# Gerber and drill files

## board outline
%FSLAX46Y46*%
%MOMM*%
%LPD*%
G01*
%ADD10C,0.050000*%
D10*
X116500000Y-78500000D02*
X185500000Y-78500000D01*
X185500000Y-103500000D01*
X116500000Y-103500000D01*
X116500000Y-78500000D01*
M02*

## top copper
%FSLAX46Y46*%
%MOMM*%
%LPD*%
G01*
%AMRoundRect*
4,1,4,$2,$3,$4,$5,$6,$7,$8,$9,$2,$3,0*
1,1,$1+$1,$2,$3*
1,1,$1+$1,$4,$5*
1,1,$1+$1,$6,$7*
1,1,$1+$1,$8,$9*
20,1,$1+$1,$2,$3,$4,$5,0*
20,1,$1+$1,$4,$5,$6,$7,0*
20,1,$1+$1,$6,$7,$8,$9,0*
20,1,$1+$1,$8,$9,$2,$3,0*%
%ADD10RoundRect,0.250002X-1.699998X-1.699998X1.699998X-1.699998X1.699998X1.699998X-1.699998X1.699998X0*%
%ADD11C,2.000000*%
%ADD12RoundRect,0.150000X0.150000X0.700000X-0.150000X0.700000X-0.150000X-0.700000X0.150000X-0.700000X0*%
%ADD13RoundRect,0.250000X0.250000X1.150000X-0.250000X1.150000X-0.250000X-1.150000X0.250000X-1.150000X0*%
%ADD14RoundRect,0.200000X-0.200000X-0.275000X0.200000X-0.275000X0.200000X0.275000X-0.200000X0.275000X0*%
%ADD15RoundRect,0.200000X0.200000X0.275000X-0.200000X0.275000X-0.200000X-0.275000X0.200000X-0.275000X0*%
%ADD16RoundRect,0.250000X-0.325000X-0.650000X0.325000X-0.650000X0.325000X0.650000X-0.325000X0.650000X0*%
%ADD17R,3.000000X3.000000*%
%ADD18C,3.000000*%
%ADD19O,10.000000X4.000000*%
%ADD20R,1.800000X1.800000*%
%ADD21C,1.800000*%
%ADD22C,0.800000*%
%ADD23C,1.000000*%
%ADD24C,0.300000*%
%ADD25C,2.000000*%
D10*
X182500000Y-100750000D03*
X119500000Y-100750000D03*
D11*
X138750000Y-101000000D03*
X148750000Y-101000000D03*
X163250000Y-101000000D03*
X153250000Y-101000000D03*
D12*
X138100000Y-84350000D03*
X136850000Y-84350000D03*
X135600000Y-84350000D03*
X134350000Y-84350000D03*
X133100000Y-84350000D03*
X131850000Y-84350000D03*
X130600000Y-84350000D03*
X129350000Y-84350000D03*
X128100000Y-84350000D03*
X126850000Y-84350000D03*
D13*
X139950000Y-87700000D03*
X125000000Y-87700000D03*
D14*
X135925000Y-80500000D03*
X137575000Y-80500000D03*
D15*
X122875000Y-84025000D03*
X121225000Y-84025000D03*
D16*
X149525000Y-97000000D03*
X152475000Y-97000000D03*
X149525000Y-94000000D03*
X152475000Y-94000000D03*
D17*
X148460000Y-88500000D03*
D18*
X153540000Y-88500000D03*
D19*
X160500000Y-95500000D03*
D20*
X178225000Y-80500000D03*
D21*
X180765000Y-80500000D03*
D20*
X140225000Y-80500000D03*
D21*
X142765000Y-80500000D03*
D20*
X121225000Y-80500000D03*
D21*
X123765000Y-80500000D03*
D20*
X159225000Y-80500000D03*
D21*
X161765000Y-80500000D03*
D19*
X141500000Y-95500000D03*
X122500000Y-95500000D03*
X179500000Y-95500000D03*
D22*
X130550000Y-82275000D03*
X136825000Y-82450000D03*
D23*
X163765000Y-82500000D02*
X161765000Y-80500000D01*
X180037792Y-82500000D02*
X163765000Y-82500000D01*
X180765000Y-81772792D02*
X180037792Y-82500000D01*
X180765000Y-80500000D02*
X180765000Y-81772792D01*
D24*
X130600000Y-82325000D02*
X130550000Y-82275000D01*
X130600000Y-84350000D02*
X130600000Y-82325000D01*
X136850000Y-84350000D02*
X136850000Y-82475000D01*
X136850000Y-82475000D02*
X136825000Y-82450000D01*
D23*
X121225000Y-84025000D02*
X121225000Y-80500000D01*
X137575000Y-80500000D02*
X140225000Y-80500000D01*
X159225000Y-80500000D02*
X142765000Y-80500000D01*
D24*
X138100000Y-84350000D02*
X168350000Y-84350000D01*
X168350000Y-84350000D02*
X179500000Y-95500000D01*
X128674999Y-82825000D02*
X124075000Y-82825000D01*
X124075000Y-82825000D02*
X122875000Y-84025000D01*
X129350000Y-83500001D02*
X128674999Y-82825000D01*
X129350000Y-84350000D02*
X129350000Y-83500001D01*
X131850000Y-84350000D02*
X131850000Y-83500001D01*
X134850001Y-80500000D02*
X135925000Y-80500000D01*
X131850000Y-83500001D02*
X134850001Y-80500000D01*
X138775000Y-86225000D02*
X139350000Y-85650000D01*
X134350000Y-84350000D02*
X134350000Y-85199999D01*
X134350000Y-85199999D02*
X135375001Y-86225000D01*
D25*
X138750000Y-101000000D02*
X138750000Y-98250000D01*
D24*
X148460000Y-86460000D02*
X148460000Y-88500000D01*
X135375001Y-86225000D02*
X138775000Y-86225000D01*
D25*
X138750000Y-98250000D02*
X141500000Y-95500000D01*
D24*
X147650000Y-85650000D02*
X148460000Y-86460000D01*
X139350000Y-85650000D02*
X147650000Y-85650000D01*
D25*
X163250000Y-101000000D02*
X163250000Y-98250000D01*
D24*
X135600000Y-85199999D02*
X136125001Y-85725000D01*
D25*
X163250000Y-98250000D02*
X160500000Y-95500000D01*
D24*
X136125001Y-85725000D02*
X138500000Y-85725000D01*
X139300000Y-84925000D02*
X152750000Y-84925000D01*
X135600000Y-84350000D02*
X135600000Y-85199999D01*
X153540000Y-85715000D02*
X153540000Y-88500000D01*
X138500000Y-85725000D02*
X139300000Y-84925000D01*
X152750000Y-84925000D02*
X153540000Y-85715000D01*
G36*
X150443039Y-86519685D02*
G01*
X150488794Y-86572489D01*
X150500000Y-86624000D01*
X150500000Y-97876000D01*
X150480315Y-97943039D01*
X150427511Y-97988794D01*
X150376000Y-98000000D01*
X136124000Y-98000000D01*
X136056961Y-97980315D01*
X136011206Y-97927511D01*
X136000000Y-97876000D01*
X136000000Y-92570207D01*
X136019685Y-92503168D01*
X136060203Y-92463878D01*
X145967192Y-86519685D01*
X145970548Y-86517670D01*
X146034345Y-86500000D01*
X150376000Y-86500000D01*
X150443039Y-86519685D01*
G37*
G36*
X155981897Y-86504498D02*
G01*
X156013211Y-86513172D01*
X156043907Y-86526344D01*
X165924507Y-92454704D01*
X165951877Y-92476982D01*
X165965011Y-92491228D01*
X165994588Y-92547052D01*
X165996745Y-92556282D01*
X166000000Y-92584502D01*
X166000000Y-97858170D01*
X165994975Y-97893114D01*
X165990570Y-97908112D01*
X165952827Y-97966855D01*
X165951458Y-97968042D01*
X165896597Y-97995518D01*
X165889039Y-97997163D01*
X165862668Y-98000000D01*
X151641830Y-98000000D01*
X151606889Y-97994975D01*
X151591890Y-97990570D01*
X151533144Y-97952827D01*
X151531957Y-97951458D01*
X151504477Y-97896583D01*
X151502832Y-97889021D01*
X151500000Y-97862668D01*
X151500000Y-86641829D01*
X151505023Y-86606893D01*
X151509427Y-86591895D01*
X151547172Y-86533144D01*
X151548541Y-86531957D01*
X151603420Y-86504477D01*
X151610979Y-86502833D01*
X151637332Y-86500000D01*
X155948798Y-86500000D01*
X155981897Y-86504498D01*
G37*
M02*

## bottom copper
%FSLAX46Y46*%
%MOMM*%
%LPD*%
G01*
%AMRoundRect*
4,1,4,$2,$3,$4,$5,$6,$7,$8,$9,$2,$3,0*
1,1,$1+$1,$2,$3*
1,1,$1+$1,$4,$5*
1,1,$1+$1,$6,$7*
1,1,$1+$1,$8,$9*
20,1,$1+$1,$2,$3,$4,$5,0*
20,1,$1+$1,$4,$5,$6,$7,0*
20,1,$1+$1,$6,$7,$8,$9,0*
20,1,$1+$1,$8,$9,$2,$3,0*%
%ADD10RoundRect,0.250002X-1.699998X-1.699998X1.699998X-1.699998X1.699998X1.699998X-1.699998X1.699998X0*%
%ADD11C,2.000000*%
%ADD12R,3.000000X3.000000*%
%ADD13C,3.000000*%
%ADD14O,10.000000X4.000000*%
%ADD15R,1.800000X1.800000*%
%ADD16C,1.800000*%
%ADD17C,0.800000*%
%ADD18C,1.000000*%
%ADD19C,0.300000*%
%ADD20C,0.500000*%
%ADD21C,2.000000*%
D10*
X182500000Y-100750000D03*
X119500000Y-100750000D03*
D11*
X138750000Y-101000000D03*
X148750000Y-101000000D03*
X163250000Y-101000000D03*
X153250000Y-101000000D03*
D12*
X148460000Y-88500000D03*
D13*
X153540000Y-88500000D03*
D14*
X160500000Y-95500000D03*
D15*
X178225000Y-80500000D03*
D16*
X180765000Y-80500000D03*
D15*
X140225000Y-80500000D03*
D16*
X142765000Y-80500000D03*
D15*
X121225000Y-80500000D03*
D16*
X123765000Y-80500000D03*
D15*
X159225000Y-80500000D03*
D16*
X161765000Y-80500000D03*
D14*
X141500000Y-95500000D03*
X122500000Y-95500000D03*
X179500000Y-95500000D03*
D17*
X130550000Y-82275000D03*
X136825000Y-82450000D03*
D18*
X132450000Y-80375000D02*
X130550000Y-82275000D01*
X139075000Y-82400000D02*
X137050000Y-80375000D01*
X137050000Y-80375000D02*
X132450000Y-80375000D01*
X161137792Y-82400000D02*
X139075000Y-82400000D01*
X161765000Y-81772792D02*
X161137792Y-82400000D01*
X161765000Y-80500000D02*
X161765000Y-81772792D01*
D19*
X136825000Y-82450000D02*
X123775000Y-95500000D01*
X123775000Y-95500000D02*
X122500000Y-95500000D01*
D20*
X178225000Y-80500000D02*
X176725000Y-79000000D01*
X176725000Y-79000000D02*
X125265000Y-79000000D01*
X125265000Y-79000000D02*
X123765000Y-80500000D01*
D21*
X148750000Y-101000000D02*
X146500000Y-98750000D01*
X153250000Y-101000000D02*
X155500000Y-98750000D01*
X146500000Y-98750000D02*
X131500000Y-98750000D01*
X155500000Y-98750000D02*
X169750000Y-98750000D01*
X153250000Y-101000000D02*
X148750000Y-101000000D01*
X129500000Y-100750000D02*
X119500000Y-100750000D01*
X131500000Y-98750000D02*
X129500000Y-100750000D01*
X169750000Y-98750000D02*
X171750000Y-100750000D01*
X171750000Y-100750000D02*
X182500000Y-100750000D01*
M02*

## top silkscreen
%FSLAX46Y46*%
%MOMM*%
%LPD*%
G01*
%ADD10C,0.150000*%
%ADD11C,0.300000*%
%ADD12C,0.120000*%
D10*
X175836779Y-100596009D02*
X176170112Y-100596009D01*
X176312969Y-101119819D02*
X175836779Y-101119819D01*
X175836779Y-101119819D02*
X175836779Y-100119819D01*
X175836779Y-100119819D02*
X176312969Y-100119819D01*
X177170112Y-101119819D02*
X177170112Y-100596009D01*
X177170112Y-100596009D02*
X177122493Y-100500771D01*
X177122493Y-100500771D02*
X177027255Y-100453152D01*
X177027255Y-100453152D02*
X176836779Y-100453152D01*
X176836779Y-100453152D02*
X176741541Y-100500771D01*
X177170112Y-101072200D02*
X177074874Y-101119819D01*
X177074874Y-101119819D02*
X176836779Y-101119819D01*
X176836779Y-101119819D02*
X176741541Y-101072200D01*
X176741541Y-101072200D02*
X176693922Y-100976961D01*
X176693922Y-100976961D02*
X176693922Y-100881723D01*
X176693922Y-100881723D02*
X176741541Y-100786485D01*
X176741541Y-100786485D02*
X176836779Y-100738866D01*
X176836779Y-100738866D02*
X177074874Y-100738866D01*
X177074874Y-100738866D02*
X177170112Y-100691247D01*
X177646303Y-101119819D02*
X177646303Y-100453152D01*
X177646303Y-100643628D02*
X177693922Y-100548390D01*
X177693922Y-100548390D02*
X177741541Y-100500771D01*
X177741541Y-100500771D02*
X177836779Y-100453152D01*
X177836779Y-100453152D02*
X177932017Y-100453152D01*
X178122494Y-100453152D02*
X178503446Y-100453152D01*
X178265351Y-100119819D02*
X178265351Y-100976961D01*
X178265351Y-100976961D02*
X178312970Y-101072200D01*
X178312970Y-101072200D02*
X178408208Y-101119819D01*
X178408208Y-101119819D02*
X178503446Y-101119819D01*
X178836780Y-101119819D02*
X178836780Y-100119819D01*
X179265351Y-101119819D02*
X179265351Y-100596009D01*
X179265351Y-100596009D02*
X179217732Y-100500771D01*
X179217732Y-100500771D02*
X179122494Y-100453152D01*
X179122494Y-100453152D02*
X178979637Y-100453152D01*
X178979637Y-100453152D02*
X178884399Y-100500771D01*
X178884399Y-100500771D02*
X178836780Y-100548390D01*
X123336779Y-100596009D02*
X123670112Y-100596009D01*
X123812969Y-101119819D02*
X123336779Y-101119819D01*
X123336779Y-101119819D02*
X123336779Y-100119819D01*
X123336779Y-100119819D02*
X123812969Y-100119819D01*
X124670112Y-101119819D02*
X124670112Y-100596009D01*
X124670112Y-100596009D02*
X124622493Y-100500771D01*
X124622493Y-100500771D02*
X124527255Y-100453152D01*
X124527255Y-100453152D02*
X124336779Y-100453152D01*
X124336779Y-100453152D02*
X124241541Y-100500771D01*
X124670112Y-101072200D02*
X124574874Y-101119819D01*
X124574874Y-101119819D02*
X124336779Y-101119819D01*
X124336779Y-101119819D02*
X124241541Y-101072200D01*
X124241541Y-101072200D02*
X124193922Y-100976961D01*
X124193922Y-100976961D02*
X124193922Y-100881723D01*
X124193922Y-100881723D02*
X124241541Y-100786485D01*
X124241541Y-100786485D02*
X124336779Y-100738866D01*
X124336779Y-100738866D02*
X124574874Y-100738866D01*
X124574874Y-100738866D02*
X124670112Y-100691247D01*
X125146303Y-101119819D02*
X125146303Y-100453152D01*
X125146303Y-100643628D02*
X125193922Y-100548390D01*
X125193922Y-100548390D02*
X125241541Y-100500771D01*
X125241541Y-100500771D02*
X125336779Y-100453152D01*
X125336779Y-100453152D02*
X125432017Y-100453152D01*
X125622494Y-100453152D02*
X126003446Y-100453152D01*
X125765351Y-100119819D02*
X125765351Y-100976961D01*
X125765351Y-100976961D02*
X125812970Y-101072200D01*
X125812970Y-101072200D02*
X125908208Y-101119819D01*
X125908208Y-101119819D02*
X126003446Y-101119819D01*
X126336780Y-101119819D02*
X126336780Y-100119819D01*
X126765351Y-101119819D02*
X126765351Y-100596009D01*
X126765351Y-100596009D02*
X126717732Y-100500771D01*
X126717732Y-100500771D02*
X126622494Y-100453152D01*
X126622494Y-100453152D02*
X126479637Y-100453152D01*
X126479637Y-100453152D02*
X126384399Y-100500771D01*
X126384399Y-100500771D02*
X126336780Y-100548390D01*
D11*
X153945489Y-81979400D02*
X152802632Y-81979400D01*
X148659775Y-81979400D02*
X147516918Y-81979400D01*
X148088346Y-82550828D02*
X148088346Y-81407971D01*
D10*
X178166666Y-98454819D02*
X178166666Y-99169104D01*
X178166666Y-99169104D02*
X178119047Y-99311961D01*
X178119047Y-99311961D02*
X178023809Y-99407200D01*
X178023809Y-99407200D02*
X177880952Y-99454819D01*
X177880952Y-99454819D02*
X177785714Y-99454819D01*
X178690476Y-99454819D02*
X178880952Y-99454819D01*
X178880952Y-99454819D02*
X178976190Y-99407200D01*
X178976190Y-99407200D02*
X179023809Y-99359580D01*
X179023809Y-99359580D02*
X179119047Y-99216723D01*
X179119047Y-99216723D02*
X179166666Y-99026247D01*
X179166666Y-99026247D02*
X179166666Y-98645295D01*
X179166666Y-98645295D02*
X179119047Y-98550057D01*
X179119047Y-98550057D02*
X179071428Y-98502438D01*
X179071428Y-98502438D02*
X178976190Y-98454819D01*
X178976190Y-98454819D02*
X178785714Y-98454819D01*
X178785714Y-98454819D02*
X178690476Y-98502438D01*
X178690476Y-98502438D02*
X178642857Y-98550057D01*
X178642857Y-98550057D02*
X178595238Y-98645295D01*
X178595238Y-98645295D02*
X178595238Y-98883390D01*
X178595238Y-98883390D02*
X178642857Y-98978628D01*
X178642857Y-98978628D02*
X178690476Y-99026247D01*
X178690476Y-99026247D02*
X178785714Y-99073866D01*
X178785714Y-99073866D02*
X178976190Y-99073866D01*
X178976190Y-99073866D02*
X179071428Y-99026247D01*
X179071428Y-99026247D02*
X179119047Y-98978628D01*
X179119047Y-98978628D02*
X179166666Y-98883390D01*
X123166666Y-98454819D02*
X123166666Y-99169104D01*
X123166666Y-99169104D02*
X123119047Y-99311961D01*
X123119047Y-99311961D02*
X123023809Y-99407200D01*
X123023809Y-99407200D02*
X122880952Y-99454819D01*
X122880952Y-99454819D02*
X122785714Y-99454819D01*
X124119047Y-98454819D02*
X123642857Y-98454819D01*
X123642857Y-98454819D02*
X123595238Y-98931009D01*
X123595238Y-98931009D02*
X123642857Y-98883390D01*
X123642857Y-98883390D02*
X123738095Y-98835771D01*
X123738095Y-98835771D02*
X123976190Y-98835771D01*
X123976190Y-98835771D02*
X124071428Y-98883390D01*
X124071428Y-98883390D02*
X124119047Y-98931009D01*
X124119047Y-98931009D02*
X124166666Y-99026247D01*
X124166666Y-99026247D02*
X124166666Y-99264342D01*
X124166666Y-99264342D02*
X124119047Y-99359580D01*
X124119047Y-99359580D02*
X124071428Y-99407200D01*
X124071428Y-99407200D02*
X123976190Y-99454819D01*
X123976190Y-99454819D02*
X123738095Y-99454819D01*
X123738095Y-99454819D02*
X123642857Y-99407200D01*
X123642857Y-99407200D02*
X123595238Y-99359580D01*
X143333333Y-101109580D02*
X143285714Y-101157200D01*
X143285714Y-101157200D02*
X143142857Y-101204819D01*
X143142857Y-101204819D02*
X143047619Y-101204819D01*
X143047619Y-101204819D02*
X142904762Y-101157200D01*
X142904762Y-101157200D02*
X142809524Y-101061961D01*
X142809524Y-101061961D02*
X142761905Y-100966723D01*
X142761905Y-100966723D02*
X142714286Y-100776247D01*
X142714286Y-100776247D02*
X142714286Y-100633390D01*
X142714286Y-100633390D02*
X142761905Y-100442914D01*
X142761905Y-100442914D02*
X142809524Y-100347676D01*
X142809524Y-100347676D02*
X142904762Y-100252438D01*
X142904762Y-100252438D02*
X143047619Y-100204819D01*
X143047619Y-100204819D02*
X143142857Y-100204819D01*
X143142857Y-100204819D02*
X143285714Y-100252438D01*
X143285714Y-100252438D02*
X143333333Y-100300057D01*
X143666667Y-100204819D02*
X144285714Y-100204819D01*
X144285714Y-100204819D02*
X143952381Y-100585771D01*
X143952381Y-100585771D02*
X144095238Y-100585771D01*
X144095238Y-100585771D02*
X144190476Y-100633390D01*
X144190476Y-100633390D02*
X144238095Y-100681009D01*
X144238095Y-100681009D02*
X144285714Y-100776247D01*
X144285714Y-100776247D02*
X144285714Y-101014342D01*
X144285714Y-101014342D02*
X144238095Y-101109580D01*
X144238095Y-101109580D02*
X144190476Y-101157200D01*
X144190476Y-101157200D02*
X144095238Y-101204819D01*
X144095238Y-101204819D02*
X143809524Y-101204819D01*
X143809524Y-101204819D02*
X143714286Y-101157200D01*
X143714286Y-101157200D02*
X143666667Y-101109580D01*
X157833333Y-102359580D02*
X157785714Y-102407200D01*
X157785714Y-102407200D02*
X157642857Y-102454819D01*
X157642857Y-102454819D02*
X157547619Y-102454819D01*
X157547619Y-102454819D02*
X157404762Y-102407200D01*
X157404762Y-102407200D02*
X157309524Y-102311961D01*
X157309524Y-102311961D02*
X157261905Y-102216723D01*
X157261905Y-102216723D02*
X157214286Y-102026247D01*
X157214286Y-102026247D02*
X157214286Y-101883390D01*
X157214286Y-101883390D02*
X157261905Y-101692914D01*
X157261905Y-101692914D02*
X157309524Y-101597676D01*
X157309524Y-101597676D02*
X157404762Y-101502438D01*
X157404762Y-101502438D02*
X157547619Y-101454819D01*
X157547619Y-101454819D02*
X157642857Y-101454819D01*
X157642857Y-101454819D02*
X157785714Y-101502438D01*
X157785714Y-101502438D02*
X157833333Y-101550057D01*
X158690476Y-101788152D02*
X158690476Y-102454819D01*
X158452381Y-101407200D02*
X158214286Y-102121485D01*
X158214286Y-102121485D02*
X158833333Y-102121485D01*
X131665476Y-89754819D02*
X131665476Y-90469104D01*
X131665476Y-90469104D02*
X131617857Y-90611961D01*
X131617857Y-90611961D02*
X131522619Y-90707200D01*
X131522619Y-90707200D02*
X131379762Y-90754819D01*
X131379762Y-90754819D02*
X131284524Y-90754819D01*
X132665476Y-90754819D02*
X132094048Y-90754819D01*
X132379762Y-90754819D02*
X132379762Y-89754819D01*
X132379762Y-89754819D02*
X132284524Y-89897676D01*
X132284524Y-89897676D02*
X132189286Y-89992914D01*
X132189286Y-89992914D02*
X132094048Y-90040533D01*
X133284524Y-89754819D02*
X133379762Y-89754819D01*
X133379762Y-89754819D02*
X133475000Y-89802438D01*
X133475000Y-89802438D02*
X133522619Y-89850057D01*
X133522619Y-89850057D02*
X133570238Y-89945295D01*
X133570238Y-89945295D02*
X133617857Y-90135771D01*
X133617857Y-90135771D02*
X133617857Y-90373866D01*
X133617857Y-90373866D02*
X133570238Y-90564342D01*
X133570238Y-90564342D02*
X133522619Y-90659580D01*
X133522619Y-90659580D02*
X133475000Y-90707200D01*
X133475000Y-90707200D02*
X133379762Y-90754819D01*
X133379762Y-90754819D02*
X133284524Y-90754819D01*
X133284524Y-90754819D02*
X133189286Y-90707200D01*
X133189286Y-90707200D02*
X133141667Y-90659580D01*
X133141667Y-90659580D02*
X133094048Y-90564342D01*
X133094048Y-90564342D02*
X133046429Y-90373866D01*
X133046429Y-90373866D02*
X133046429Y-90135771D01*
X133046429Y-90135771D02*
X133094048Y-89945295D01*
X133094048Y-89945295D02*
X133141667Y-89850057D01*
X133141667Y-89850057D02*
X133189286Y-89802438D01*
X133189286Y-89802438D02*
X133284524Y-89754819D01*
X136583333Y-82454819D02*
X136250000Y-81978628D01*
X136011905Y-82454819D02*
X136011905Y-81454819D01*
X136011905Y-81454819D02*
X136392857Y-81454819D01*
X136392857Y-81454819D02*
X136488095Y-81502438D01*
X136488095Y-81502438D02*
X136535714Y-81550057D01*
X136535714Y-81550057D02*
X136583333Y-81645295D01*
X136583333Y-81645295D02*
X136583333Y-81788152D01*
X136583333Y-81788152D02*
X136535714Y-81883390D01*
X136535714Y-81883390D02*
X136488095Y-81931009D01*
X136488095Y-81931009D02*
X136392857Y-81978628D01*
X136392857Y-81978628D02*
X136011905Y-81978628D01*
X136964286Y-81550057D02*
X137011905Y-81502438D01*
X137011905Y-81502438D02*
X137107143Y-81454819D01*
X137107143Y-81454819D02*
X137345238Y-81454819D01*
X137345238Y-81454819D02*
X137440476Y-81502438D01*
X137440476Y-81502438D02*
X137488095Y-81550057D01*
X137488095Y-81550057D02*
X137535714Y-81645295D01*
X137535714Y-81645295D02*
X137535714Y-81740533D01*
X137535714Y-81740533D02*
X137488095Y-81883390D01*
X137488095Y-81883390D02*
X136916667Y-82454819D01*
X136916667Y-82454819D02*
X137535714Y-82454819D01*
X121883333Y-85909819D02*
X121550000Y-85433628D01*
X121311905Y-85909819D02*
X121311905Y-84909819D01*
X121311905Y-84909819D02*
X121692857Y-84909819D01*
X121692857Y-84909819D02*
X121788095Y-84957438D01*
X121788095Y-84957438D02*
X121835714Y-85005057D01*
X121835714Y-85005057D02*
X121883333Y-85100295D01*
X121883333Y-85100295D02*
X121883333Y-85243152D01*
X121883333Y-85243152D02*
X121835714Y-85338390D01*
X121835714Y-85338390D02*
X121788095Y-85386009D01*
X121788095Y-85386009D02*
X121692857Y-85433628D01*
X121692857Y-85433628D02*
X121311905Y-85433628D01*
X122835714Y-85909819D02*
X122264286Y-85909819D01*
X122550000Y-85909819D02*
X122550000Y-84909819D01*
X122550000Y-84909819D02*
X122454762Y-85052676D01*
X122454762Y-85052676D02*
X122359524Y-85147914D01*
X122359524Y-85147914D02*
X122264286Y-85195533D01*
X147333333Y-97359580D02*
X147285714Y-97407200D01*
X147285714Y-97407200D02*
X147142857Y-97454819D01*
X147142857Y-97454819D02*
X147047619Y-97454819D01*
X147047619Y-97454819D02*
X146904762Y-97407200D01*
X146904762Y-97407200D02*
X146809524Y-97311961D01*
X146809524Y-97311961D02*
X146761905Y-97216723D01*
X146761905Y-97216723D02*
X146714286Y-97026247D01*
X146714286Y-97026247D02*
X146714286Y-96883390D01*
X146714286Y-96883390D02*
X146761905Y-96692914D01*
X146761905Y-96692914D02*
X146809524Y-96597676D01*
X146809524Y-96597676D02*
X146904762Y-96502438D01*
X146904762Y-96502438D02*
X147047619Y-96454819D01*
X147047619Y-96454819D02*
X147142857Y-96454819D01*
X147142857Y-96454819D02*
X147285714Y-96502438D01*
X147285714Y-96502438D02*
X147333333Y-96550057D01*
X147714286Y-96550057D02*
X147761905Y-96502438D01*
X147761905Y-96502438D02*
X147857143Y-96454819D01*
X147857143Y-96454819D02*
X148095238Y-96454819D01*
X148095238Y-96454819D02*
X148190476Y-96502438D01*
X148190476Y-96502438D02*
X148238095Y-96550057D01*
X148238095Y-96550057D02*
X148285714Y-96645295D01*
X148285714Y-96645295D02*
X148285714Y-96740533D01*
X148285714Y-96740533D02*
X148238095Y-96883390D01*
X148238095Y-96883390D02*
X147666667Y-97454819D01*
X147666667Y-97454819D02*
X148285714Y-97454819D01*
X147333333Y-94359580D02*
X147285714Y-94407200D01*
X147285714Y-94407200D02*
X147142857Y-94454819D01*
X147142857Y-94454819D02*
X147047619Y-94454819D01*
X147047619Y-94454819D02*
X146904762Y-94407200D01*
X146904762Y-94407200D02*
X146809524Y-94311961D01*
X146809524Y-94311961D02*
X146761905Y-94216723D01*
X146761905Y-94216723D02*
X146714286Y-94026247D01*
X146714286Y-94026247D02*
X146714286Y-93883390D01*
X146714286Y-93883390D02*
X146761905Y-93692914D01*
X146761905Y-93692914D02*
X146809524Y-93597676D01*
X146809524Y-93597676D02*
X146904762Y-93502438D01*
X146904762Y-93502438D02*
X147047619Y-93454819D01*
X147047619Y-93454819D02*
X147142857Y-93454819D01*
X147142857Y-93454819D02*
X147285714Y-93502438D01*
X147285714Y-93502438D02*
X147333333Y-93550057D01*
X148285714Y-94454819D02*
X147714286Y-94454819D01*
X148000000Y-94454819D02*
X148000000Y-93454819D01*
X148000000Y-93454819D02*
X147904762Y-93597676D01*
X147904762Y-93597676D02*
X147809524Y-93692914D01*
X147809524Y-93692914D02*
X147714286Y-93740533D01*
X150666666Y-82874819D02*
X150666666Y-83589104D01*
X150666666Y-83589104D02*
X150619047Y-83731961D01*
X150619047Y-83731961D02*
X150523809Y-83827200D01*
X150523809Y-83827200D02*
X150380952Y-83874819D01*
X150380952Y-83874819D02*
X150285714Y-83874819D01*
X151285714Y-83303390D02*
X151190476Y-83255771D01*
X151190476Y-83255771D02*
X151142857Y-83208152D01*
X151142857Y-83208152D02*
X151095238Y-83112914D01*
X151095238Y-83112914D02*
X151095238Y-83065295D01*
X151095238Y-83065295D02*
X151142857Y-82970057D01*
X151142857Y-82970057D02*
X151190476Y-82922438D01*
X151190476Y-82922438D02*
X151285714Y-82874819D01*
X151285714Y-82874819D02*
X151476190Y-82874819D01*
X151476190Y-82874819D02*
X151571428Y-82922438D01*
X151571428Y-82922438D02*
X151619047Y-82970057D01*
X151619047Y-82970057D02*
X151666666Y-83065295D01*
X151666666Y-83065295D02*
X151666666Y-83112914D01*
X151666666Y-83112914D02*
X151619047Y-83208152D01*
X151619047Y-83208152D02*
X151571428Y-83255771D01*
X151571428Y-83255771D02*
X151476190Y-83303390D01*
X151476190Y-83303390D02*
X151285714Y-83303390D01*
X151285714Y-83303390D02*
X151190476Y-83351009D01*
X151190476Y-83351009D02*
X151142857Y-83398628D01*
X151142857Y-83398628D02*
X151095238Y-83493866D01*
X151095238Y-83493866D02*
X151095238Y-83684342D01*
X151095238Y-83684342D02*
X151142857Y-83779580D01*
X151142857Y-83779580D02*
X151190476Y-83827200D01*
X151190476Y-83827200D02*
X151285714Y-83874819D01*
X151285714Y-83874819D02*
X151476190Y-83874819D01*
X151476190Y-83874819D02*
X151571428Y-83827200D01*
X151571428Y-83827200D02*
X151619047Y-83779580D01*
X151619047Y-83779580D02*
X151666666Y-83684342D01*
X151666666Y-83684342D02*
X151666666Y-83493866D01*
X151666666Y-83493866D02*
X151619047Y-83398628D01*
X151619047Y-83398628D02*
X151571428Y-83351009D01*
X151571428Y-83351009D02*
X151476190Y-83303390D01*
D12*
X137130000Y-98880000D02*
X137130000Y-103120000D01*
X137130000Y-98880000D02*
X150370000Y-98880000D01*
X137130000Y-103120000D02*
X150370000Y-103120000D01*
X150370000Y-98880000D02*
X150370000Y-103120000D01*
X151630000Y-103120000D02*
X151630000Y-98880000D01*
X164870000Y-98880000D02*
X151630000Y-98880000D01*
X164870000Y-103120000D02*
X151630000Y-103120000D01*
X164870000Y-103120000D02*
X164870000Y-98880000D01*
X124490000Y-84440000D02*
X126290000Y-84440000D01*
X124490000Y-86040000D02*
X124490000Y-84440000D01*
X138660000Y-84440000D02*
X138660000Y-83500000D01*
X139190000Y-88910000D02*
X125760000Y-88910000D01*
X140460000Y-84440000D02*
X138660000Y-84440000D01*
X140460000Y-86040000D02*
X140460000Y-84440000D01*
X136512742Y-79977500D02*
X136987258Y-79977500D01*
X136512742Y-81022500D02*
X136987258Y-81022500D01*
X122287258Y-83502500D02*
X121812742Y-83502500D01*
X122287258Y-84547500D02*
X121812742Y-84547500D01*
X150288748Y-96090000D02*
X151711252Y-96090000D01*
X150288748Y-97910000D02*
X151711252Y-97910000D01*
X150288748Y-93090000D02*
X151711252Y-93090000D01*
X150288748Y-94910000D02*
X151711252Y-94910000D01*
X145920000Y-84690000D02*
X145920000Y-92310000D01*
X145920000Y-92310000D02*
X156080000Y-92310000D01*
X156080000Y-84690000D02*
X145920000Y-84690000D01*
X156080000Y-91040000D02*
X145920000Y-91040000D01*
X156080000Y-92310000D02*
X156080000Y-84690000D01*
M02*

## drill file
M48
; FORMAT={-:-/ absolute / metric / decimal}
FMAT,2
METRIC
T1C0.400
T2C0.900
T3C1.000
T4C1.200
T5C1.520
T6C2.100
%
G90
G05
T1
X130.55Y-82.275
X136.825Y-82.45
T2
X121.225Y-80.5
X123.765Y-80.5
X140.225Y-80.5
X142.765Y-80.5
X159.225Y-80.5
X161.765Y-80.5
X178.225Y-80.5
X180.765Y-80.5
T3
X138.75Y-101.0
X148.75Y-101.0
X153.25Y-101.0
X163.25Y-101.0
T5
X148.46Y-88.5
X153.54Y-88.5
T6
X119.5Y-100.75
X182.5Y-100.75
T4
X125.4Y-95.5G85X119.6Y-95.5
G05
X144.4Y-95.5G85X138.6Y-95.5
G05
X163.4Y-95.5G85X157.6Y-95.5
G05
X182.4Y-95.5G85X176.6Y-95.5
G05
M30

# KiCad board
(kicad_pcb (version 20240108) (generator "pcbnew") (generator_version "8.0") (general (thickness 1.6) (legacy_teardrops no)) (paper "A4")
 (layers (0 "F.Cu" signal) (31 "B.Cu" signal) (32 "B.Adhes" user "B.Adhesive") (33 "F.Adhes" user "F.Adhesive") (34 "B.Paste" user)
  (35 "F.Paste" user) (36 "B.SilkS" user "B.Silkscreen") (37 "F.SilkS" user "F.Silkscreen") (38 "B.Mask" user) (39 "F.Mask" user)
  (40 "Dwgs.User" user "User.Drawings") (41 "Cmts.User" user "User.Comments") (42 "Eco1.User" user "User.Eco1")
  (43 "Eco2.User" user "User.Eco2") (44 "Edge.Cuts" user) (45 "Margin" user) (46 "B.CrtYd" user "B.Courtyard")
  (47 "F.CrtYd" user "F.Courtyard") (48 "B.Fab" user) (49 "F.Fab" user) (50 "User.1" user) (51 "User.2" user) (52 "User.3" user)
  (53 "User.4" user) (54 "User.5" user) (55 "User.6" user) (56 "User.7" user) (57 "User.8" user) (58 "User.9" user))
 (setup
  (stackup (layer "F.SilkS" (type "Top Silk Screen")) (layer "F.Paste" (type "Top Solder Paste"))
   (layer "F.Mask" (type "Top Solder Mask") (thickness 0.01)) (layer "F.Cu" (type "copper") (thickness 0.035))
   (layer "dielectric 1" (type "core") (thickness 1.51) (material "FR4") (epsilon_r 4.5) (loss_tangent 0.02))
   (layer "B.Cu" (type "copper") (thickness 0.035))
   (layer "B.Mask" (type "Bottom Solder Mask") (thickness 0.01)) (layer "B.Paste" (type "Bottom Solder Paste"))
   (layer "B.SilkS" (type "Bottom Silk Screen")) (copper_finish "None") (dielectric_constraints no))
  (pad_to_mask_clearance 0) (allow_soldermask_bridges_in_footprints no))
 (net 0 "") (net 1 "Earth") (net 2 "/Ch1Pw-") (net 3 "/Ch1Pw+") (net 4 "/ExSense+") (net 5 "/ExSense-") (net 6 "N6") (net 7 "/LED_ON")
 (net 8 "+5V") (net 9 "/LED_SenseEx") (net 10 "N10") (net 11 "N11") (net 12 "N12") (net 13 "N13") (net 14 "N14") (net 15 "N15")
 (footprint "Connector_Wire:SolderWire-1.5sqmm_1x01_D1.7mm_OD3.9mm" (layer "F.Cu") (at 182.5 100.75)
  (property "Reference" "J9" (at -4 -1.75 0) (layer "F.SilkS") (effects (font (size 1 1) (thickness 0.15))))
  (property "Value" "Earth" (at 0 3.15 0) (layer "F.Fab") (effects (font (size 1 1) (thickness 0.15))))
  (pad "1" thru_hole roundrect (at 0 0) (size 3.9 3.9) (drill 2.1) (layers "*.Cu" "*.Mask") (remove_unused_layers no)
   (roundrect_rratio 0.064103) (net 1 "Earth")))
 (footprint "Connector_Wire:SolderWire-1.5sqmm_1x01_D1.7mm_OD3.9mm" (layer "F.Cu") (at 119.5 100.75)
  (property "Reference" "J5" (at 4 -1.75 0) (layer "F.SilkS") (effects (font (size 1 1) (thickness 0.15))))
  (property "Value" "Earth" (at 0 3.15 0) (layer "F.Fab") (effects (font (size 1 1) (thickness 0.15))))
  (pad "1" thru_hole roundrect (at 0 0) (size 3.9 3.9) (drill 2.1) (layers "*.Cu" "*.Mask") (remove_unused_layers no)
   (roundrect_rratio 0.064103) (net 1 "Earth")))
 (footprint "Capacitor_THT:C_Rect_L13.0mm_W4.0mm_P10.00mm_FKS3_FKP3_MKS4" (layer "F.Cu") (at 138.75 101)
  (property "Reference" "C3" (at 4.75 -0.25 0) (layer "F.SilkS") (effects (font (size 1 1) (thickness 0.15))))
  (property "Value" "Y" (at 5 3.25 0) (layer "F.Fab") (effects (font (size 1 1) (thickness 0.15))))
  (fp_line (start -1.62 -2.12) (end -1.62 2.12) (stroke (width 0.12) (type solid)) (layer "F.SilkS"))
  (fp_line (start -1.62 -2.12) (end 11.62 -2.12) (stroke (width 0.12) (type solid)) (layer "F.SilkS"))
  (fp_line (start -1.62 2.12) (end 11.62 2.12) (stroke (width 0.12) (type solid)) (layer "F.SilkS"))
  (fp_line (start 11.62 -2.12) (end 11.62 2.12) (stroke (width 0.12) (type solid)) (layer "F.SilkS"))
  (pad "1" thru_hole circle (at 0 0) (size 2 2) (drill 1) (layers "*.Cu" "*.Mask") (remove_unused_layers no) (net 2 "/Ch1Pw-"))
  (pad "2" thru_hole circle (at 10 0) (size 2 2) (drill 1) (layers "*.Cu" "*.Mask") (remove_unused_layers no) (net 1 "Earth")))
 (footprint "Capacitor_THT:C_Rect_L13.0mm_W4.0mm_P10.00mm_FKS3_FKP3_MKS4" (layer "F.Cu") (at 163.25 101 180)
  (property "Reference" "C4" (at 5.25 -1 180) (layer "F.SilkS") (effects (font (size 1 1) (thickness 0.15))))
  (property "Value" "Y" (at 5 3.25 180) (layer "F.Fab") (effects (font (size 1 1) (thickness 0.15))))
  (fp_line (start 11.62 -2.12) (end 11.62 2.12) (stroke (width 0.12) (type solid)) (layer "F.SilkS"))
  (fp_line (start -1.62 2.12) (end 11.62 2.12) (stroke (width 0.12) (type solid)) (layer "F.SilkS"))
  (fp_line (start -1.62 -2.12) (end 11.62 -2.12) (stroke (width 0.12) (type solid)) (layer "F.SilkS"))
  (fp_line (start -1.62 -2.12) (end -1.62 2.12) (stroke (width 0.12) (type solid)) (layer "F.SilkS"))
  (pad "1" thru_hole circle (at 0 0 180) (size 2 2) (drill 1) (layers "*.Cu" "*.Mask") (remove_unused_layers no) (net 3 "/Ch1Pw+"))
  (pad "2" thru_hole circle (at 10 0 180) (size 2 2) (drill 1) (layers "*.Cu" "*.Mask") (remove_unused_layers no) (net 1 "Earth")))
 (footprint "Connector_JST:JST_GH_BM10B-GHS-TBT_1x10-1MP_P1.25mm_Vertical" (layer "F.Cu") (at 132.475 86.3 180)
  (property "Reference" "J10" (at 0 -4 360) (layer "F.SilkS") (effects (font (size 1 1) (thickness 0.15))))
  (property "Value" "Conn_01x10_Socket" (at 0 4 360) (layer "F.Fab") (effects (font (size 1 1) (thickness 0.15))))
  (fp_line (start 7.985 1.86) (end 6.185 1.86) (stroke (width 0.12) (type solid)) (layer "F.SilkS"))
  (fp_line (start 7.985 0.26) (end 7.985 1.86) (stroke (width 0.12) (type solid)) (layer "F.SilkS"))
  (fp_line (start -6.185 1.86) (end -6.185 2.8) (stroke (width 0.12) (type solid)) (layer "F.SilkS"))
  (fp_line (start -6.715 -2.61) (end 6.715 -2.61) (stroke (width 0.12) (type solid)) (layer "F.SilkS"))
  (fp_line (start -7.985 1.86) (end -6.185 1.86) (stroke (width 0.12) (type solid)) (layer "F.SilkS"))
  (fp_line (start -7.985 0.26) (end -7.985 1.86) (stroke (width 0.12) (type solid)) (layer "F.SilkS"))
  (pad "1" smd roundrect (at -5.625 1.95 180) (size 0.6 1.7) (layers "F.Cu" "F.Paste" "F.Mask") (roundrect_rratio 0.25) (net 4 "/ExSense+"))
  (pad "2" smd roundrect (at -4.375 1.95 180) (size 0.6 1.7) (layers "F.Cu" "F.Paste" "F.Mask") (roundrect_rratio 0.25) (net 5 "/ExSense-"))
  (pad "3" smd roundrect (at -3.125 1.95 180) (size 0.6 1.7) (layers "F.Cu" "F.Paste" "F.Mask") (roundrect_rratio 0.25) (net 3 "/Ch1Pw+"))
  (pad "4" smd roundrect (at -1.875 1.95 180) (size 0.6 1.7) (layers "F.Cu" "F.Paste" "F.Mask") (roundrect_rratio 0.25) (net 2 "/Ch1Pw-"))
  (pad "5" smd roundrect (at -0.625 1.95 180) (size 0.6 1.7) (layers "F.Cu" "F.Paste" "F.Mask") (roundrect_rratio 0.25) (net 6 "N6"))
  (pad "6" smd roundrect (at 0.625 1.95 180) (size 0.6 1.7) (layers "F.Cu" "F.Paste" "F.Mask") (roundrect_rratio 0.25) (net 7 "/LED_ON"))
  (pad "7" smd roundrect (at 1.875 1.95 180) (size 0.6 1.7) (layers "F.Cu" "F.Paste" "F.Mask") (roundrect_rratio 0.25) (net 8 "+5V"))
  (pad "8" smd roundrect (at 3.125 1.95 180) (size 0.6 1.7) (layers "F.Cu" "F.Paste" "F.Mask") (roundrect_rratio 0.25)
   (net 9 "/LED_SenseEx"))
  (pad "9" smd roundrect (at 4.375 1.95 180) (size 0.6 1.7) (layers "F.Cu" "F.Paste" "F.Mask") (roundrect_rratio 0.25) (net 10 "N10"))
  (pad "10" smd roundrect (at 5.625 1.95 180) (size 0.6 1.7) (layers "F.Cu" "F.Paste" "F.Mask") (roundrect_rratio 0.25) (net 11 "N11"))
  (pad "MP" smd roundrect (at -7.475 -1.4 180) (size 1 2.8) (layers "F.Cu" "F.Paste" "F.Mask") (roundrect_rratio 0.25))
  (pad "MP" smd roundrect (at 7.475 -1.4 180) (size 1 2.8) (layers "F.Cu" "F.Paste" "F.Mask") (roundrect_rratio 0.25)))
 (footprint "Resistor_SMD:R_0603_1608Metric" (layer "F.Cu") (at 136.75 80.5)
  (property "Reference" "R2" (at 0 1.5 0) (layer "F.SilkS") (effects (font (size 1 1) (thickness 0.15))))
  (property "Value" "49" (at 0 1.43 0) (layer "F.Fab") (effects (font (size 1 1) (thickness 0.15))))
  (fp_line (start -0.237258 -0.5225) (end 0.237258 -0.5225) (stroke (width 0.12) (type solid)) (layer "F.SilkS"))
  (fp_line (start -0.237258 0.5225) (end 0.237258 0.5225) (stroke (width 0.12) (type solid)) (layer "F.SilkS"))
  (pad "1" smd roundrect (at -0.825 0) (size 0.8 0.95) (layers "F.Cu" "F.Paste" "F.Mask") (roundrect_rratio 0.25) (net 7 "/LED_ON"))
  (pad "2" smd roundrect (at 0.825 0) (size 0.8 0.95) (layers "F.Cu" "F.Paste" "F.Mask") (roundrect_rratio 0.25) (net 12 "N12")))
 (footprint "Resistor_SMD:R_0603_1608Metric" (layer "F.Cu") (at 122.05 84.025 180)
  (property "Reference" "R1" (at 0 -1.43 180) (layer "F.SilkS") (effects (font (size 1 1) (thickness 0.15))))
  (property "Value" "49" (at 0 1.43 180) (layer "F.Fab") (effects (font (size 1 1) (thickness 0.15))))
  (fp_line (start -0.237258 0.5225) (end 0.237258 0.5225) (stroke (width 0.12) (type solid)) (layer "F.SilkS"))
  (fp_line (start -0.237258 -0.5225) (end 0.237258 -0.5225) (stroke (width 0.12) (type solid)) (layer "F.SilkS"))
  (pad "1" smd roundrect (at -0.825 0 180) (size 0.8 0.95) (layers "F.Cu" "F.Paste" "F.Mask") (roundrect_rratio 0.25) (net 9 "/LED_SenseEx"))
  (pad "2" smd roundrect (at 0.825 0 180) (size 0.8 0.95) (layers "F.Cu" "F.Paste" "F.Mask") (roundrect_rratio 0.25) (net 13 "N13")))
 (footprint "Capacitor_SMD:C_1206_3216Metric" (layer "F.Cu") (at 151 97)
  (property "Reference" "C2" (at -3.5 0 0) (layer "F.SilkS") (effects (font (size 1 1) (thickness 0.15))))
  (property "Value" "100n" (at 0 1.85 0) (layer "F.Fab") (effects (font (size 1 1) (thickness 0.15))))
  (fp_line (start -0.711252 -0.91) (end 0.711252 -0.91) (stroke (width 0.12) (type solid)) (layer "F.SilkS"))
  (fp_line (start -0.711252 0.91) (end 0.711252 0.91) (stroke (width 0.12) (type solid)) (layer "F.SilkS"))
  (pad "1" smd roundrect (at -1.475 0) (size 1.15 1.8) (layers "F.Cu" "F.Paste" "F.Mask") (roundrect_rratio 0.217391) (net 2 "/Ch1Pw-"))
  (pad "2" smd roundrect (at 1.475 0) (size 1.15 1.8) (layers "F.Cu" "F.Paste" "F.Mask") (roundrect_rratio 0.217391) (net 3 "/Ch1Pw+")))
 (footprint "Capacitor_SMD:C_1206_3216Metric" (layer "F.Cu") (at 151 94)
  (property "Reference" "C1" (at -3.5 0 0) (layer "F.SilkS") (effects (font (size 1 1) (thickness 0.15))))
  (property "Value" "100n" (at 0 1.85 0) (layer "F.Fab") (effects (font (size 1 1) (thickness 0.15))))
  (fp_line (start -0.711252 -0.91) (end 0.711252 -0.91) (stroke (width 0.12) (type solid)) (layer "F.SilkS"))
  (fp_line (start -0.711252 0.91) (end 0.711252 0.91) (stroke (width 0.12) (type solid)) (layer "F.SilkS"))
  (pad "1" smd roundrect (at -1.475 0) (size 1.15 1.8) (layers "F.Cu" "F.Paste" "F.Mask") (roundrect_rratio 0.217391) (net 2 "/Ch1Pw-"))
  (pad "2" smd roundrect (at 1.475 0) (size 1.15 1.8) (layers "F.Cu" "F.Paste" "F.Mask") (roundrect_rratio 0.217391) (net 3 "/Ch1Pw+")))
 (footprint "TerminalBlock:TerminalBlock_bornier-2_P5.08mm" (layer "F.Cu") (at 148.46 88.5)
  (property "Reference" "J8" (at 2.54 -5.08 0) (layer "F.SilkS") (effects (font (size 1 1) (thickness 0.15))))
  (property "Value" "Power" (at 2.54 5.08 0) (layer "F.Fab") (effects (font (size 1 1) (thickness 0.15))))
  (fp_line (start -2.54 -3.81) (end -2.54 3.81) (stroke (width 0.12) (type solid)) (layer "F.SilkS"))
  (fp_line (start -2.54 3.81) (end 7.62 3.81) (stroke (width 0.12) (type solid)) (layer "F.SilkS"))
  (fp_line (start 7.62 -3.81) (end -2.54 -3.81) (stroke (width 0.12) (type solid)) (layer "F.SilkS"))
  (fp_line (start 7.62 2.54) (end -2.54 2.54) (stroke (width 0.12) (type solid)) (layer "F.SilkS"))
  (fp_line (start 7.62 3.81) (end 7.62 -3.81) (stroke (width 0.12) (type solid)) (layer "F.SilkS"))
  (pad "1" thru_hole rect (at 0 0) (size 3 3) (drill 1.52) (layers "*.Cu" "*.Mask") (remove_unused_layers no) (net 2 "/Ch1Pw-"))
  (pad "2" thru_hole circle (at 5.08 0) (size 3 3) (drill 1.52) (layers "*.Cu" "*.Mask") (remove_unused_layers no) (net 3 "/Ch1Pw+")))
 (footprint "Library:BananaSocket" (layer "B.Cu") (at 160.5 95.5 180)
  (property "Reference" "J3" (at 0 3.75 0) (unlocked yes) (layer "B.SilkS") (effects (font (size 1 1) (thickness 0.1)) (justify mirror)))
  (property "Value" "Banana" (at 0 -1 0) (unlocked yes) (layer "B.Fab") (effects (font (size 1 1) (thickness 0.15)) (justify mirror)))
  (pad "1" thru_hole oval (at 0 0 180) (size 10 4) (drill oval 7 1.2) (layers "*.Cu" "*.Mask") (remove_unused_layers no) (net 3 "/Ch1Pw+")))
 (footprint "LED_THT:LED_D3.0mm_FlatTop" (layer "B.Cu") (at 178.225 80.5)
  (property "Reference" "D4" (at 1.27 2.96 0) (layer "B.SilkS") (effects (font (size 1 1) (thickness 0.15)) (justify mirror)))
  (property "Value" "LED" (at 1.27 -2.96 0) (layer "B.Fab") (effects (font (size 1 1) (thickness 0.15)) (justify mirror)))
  (pad "1" thru_hole rect (at 0 0) (size 1.8 1.8) (drill 0.9) (layers "*.Cu" "*.Mask") (remove_unused_layers no) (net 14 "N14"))
  (pad "2" thru_hole circle (at 2.54 0) (size 1.8 1.8) (drill 0.9) (layers "*.Cu" "*.Mask") (remove_unused_layers no) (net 8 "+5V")))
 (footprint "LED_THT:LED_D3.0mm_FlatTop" (layer "B.Cu") (at 140.225 80.5)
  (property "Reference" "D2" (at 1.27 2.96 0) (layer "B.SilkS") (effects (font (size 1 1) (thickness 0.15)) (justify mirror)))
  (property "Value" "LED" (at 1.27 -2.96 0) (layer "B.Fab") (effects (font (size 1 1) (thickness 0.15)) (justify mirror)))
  (pad "1" thru_hole rect (at 0 0) (size 1.8 1.8) (drill 0.9) (layers "*.Cu" "*.Mask") (remove_unused_layers no) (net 12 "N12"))
  (pad "2" thru_hole circle (at 2.54 0) (size 1.8 1.8) (drill 0.9) (layers "*.Cu" "*.Mask") (remove_unused_layers no) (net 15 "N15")))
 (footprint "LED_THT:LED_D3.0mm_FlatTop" (layer "B.Cu") (at 121.225 80.5)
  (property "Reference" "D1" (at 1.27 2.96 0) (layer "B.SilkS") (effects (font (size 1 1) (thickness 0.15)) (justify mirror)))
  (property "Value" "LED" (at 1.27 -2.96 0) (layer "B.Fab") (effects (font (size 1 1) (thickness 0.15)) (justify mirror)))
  (pad "1" thru_hole rect (at 0 0) (size 1.8 1.8) (drill 0.9) (layers "*.Cu" "*.Mask") (remove_unused_layers no) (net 13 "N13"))
  (pad "2" thru_hole circle (at 2.54 0) (size 1.8 1.8) (drill 0.9) (layers "*.Cu" "*.Mask") (remove_unused_layers no) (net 14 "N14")))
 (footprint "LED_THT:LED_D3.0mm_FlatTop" (layer "B.Cu") (at 159.225 80.5)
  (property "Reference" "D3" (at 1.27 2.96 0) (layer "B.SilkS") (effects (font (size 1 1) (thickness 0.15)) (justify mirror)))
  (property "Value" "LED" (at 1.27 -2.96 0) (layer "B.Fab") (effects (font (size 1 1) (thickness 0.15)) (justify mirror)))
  (pad "1" thru_hole rect (at 0 0) (size 1.8 1.8) (drill 0.9) (layers "*.Cu" "*.Mask") (remove_unused_layers no) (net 15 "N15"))
  (pad "2" thru_hole circle (at 2.54 0) (size 1.8 1.8) (drill 0.9) (layers "*.Cu" "*.Mask") (remove_unused_layers no) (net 8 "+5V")))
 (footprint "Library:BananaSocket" (layer "B.Cu") (at 141.5 95.5 180)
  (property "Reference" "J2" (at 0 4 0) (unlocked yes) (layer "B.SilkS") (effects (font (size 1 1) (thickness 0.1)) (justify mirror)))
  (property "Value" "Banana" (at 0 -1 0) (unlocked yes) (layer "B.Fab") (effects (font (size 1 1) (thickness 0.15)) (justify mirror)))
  (pad "1" thru_hole oval (at 0 0 180) (size 10 4) (drill oval 7 1.2) (layers "*.Cu" "*.Mask") (remove_unused_layers no) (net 2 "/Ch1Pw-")))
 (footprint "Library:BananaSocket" (layer "B.Cu") (at 122.5 95.5 180)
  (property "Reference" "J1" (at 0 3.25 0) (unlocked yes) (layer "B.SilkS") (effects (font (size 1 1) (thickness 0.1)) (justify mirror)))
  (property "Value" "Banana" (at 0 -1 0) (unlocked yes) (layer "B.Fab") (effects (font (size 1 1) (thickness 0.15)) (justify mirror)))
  (pad "1" thru_hole oval (at 0 0 180) (size 10 4) (drill oval 7 1.2) (layers "*.Cu" "*.Mask") (remove_unused_layers no) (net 5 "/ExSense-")))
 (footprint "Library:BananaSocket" (layer "B.Cu") (at 179.5 95.5 180)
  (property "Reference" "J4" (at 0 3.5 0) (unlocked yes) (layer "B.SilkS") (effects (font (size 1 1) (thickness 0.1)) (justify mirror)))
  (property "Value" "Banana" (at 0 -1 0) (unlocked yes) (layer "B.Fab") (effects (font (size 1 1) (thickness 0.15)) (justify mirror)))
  (pad "1" thru_hole oval (at 0 0 180) (size 10 4) (drill oval 7 1.2) (layers "*.Cu" "*.Mask") (remove_unused_layers no) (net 4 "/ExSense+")))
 (gr_rect (start 116.5 78.5) (end 185.5 103.5) (stroke (width 0.05) (type default)) (fill none) (layer "Edge.Cuts"))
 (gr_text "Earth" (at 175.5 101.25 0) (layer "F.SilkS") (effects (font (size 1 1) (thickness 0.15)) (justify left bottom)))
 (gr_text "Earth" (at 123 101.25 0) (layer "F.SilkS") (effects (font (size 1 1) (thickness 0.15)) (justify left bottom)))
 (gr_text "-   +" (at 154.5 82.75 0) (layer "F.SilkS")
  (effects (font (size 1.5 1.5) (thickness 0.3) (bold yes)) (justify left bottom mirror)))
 (segment (start 163.765 82.5) (end 161.765 80.5) (width 1) (layer "F.Cu") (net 8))
 (segment (start 180.037792 82.5) (end 163.765 82.5) (width 1) (layer "F.Cu") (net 8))
 (segment (start 180.765 81.772792) (end 180.037792 82.5) (width 1) (layer "F.Cu") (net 8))
 (segment (start 180.765 80.5) (end 180.765 81.772792) (width 1) (layer "F.Cu") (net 8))
 (segment (start 130.6 82.325) (end 130.55 82.275) (width 0.3) (layer "F.Cu") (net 8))
 (segment (start 130.6 84.35) (end 130.6 82.325) (width 0.3) (layer "F.Cu") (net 8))
 (via (at 130.55 82.275) (size 0.8) (drill 0.4) (layers "F.Cu" "B.Cu") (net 8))
 (segment (start 132.45 80.375) (end 130.55 82.275) (width 1) (layer "B.Cu") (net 8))
 (segment (start 139.075 82.4) (end 137.05 80.375) (width 1) (layer "B.Cu") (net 8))
 (segment (start 137.05 80.375) (end 132.45 80.375) (width 1) (layer "B.Cu") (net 8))
 (segment (start 161.137792 82.4) (end 139.075 82.4) (width 1) (layer "B.Cu") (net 8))
 (segment (start 161.765 81.772792) (end 161.137792 82.4) (width 1) (layer "B.Cu") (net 8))
 (segment (start 161.765 80.5) (end 161.765 81.772792) (width 1) (layer "B.Cu") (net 8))
 (segment (start 136.85 84.35) (end 136.85 82.475) (width 0.3) (layer "F.Cu") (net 5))
 (segment (start 136.85 82.475) (end 136.825 82.45) (width 0.3) (layer "F.Cu") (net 5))
 (via (at 136.825 82.45) (size 0.8) (drill 0.4) (layers "F.Cu" "B.Cu") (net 5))
 (segment (start 136.825 82.45) (end 123.775 95.5) (width 0.3) (layer "B.Cu") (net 5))
 (segment (start 123.775 95.5) (end 122.5 95.5) (width 0.3) (layer "B.Cu") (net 5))
 (segment (start 178.225 80.5) (end 176.725 79) (width 0.5) (layer "B.Cu") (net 14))
 (segment (start 176.725 79) (end 125.265 79) (width 0.5) (layer "B.Cu") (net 14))
 (segment (start 125.265 79) (end 123.765 80.5) (width 0.5) (layer "B.Cu") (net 14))
 (segment (start 121.225 84.025) (end 121.225 80.5) (width 1) (layer "F.Cu") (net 13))
 (segment (start 137.575 80.5) (end 140.225 80.5) (width 1) (layer "F.Cu") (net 12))
 (segment (start 159.225 80.5) (end 142.765 80.5) (width 1) (layer "F.Cu") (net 15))
 (segment (start 138.1 84.35) (end 168.35 84.35) (width 0.3) (layer "F.Cu") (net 4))
 (segment (start 168.35 84.35) (end 179.5 95.5) (width 0.3) (layer "F.Cu") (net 4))
 (segment (start 128.674999 82.825) (end 124.075 82.825) (width 0.3) (layer "F.Cu") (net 9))
 (segment (start 124.075 82.825) (end 122.875 84.025) (width 0.3) (layer "F.Cu") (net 9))
 (segment (start 129.35 83.500001) (end 128.674999 82.825) (width 0.3) (layer "F.Cu") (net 9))
 (segment (start 129.35 84.35) (end 129.35 83.500001) (width 0.3) (layer "F.Cu") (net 9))
 (segment (start 131.85 84.35) (end 131.85 83.500001) (width 0.3) (layer "F.Cu") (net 7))
 (segment (start 134.850001 80.5) (end 135.925 80.5) (width 0.3) (layer "F.Cu") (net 7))
 (segment (start 131.85 83.500001) (end 134.850001 80.5) (width 0.3) (layer "F.Cu") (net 7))
 (segment (start 138.775 86.225) (end 139.35 85.65) (width 0.3) (layer "F.Cu") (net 2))
 (segment (start 134.35 84.35) (end 134.35 85.199999) (width 0.3) (layer "F.Cu") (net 2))
 (segment (start 134.35 85.199999) (end 135.375001 86.225) (width 0.3) (layer "F.Cu") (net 2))
 (segment (start 138.75 101) (end 138.75 98.25) (width 2) (layer "F.Cu") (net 2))
 (segment (start 148.46 86.46) (end 148.46 88.5) (width 0.3) (layer "F.Cu") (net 2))
 (segment (start 135.375001 86.225) (end 138.775 86.225) (width 0.3) (layer "F.Cu") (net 2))
 (segment (start 138.75 98.25) (end 141.5 95.5) (width 2) (layer "F.Cu") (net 2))
 (segment (start 147.65 85.65) (end 148.46 86.46) (width 0.3) (layer "F.Cu") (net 2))
 (segment (start 139.35 85.65) (end 147.65 85.65) (width 0.3) (layer "F.Cu") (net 2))
 (segment (start 163.25 101) (end 163.25 98.25) (width 2) (layer "F.Cu") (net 3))
 (segment (start 135.6 85.199999) (end 136.125001 85.725) (width 0.3) (layer "F.Cu") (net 3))
 (segment (start 163.25 98.25) (end 160.5 95.5) (width 2) (layer "F.Cu") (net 3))
 (segment (start 136.125001 85.725) (end 138.5 85.725) (width 0.3) (layer "F.Cu") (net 3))
 (segment (start 139.3 84.925) (end 152.75 84.925) (width 0.3) (layer "F.Cu") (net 3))
 (segment (start 135.6 84.35) (end 135.6 85.199999) (width 0.3) (layer "F.Cu") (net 3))
 (segment (start 153.54 85.715) (end 153.54 88.5) (width 0.3) (layer "F.Cu") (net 3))
 (segment (start 138.5 85.725) (end 139.3 84.925) (width 0.3) (layer "F.Cu") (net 3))
 (segment (start 152.75 84.925) (end 153.54 85.715) (width 0.3) (layer "F.Cu") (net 3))
 (segment (start 148.75 101) (end 146.5 98.75) (width 2) (layer "B.Cu") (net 1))
 (segment (start 153.25 101) (end 155.5 98.75) (width 2) (layer "B.Cu") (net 1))
 (segment (start 146.5 98.75) (end 131.5 98.75) (width 2) (layer "B.Cu") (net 1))
 (segment (start 155.5 98.75) (end 169.75 98.75) (width 2) (layer "B.Cu") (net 1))
 (segment (start 153.25 101) (end 148.75 101) (width 2) (layer "B.Cu") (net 1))
 (segment (start 129.5 100.75) (end 119.5 100.75) (width 2) (layer "B.Cu") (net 1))
 (segment (start 131.5 98.75) (end 129.5 100.75) (width 2) (layer "B.Cu") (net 1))
 (segment (start 169.75 98.75) (end 171.75 100.75) (width 2) (layer "B.Cu") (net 1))
 (segment (start 171.75 100.75) (end 182.5 100.75) (width 2) (layer "B.Cu") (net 1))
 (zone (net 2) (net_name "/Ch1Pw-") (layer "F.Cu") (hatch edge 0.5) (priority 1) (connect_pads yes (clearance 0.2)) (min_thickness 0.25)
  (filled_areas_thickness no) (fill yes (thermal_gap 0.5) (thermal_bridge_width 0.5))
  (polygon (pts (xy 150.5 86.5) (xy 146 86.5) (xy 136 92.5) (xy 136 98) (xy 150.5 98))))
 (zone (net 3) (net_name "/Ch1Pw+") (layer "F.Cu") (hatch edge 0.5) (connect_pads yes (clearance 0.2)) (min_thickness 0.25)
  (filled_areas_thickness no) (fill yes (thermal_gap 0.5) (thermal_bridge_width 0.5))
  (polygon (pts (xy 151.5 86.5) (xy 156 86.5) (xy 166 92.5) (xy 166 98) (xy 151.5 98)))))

